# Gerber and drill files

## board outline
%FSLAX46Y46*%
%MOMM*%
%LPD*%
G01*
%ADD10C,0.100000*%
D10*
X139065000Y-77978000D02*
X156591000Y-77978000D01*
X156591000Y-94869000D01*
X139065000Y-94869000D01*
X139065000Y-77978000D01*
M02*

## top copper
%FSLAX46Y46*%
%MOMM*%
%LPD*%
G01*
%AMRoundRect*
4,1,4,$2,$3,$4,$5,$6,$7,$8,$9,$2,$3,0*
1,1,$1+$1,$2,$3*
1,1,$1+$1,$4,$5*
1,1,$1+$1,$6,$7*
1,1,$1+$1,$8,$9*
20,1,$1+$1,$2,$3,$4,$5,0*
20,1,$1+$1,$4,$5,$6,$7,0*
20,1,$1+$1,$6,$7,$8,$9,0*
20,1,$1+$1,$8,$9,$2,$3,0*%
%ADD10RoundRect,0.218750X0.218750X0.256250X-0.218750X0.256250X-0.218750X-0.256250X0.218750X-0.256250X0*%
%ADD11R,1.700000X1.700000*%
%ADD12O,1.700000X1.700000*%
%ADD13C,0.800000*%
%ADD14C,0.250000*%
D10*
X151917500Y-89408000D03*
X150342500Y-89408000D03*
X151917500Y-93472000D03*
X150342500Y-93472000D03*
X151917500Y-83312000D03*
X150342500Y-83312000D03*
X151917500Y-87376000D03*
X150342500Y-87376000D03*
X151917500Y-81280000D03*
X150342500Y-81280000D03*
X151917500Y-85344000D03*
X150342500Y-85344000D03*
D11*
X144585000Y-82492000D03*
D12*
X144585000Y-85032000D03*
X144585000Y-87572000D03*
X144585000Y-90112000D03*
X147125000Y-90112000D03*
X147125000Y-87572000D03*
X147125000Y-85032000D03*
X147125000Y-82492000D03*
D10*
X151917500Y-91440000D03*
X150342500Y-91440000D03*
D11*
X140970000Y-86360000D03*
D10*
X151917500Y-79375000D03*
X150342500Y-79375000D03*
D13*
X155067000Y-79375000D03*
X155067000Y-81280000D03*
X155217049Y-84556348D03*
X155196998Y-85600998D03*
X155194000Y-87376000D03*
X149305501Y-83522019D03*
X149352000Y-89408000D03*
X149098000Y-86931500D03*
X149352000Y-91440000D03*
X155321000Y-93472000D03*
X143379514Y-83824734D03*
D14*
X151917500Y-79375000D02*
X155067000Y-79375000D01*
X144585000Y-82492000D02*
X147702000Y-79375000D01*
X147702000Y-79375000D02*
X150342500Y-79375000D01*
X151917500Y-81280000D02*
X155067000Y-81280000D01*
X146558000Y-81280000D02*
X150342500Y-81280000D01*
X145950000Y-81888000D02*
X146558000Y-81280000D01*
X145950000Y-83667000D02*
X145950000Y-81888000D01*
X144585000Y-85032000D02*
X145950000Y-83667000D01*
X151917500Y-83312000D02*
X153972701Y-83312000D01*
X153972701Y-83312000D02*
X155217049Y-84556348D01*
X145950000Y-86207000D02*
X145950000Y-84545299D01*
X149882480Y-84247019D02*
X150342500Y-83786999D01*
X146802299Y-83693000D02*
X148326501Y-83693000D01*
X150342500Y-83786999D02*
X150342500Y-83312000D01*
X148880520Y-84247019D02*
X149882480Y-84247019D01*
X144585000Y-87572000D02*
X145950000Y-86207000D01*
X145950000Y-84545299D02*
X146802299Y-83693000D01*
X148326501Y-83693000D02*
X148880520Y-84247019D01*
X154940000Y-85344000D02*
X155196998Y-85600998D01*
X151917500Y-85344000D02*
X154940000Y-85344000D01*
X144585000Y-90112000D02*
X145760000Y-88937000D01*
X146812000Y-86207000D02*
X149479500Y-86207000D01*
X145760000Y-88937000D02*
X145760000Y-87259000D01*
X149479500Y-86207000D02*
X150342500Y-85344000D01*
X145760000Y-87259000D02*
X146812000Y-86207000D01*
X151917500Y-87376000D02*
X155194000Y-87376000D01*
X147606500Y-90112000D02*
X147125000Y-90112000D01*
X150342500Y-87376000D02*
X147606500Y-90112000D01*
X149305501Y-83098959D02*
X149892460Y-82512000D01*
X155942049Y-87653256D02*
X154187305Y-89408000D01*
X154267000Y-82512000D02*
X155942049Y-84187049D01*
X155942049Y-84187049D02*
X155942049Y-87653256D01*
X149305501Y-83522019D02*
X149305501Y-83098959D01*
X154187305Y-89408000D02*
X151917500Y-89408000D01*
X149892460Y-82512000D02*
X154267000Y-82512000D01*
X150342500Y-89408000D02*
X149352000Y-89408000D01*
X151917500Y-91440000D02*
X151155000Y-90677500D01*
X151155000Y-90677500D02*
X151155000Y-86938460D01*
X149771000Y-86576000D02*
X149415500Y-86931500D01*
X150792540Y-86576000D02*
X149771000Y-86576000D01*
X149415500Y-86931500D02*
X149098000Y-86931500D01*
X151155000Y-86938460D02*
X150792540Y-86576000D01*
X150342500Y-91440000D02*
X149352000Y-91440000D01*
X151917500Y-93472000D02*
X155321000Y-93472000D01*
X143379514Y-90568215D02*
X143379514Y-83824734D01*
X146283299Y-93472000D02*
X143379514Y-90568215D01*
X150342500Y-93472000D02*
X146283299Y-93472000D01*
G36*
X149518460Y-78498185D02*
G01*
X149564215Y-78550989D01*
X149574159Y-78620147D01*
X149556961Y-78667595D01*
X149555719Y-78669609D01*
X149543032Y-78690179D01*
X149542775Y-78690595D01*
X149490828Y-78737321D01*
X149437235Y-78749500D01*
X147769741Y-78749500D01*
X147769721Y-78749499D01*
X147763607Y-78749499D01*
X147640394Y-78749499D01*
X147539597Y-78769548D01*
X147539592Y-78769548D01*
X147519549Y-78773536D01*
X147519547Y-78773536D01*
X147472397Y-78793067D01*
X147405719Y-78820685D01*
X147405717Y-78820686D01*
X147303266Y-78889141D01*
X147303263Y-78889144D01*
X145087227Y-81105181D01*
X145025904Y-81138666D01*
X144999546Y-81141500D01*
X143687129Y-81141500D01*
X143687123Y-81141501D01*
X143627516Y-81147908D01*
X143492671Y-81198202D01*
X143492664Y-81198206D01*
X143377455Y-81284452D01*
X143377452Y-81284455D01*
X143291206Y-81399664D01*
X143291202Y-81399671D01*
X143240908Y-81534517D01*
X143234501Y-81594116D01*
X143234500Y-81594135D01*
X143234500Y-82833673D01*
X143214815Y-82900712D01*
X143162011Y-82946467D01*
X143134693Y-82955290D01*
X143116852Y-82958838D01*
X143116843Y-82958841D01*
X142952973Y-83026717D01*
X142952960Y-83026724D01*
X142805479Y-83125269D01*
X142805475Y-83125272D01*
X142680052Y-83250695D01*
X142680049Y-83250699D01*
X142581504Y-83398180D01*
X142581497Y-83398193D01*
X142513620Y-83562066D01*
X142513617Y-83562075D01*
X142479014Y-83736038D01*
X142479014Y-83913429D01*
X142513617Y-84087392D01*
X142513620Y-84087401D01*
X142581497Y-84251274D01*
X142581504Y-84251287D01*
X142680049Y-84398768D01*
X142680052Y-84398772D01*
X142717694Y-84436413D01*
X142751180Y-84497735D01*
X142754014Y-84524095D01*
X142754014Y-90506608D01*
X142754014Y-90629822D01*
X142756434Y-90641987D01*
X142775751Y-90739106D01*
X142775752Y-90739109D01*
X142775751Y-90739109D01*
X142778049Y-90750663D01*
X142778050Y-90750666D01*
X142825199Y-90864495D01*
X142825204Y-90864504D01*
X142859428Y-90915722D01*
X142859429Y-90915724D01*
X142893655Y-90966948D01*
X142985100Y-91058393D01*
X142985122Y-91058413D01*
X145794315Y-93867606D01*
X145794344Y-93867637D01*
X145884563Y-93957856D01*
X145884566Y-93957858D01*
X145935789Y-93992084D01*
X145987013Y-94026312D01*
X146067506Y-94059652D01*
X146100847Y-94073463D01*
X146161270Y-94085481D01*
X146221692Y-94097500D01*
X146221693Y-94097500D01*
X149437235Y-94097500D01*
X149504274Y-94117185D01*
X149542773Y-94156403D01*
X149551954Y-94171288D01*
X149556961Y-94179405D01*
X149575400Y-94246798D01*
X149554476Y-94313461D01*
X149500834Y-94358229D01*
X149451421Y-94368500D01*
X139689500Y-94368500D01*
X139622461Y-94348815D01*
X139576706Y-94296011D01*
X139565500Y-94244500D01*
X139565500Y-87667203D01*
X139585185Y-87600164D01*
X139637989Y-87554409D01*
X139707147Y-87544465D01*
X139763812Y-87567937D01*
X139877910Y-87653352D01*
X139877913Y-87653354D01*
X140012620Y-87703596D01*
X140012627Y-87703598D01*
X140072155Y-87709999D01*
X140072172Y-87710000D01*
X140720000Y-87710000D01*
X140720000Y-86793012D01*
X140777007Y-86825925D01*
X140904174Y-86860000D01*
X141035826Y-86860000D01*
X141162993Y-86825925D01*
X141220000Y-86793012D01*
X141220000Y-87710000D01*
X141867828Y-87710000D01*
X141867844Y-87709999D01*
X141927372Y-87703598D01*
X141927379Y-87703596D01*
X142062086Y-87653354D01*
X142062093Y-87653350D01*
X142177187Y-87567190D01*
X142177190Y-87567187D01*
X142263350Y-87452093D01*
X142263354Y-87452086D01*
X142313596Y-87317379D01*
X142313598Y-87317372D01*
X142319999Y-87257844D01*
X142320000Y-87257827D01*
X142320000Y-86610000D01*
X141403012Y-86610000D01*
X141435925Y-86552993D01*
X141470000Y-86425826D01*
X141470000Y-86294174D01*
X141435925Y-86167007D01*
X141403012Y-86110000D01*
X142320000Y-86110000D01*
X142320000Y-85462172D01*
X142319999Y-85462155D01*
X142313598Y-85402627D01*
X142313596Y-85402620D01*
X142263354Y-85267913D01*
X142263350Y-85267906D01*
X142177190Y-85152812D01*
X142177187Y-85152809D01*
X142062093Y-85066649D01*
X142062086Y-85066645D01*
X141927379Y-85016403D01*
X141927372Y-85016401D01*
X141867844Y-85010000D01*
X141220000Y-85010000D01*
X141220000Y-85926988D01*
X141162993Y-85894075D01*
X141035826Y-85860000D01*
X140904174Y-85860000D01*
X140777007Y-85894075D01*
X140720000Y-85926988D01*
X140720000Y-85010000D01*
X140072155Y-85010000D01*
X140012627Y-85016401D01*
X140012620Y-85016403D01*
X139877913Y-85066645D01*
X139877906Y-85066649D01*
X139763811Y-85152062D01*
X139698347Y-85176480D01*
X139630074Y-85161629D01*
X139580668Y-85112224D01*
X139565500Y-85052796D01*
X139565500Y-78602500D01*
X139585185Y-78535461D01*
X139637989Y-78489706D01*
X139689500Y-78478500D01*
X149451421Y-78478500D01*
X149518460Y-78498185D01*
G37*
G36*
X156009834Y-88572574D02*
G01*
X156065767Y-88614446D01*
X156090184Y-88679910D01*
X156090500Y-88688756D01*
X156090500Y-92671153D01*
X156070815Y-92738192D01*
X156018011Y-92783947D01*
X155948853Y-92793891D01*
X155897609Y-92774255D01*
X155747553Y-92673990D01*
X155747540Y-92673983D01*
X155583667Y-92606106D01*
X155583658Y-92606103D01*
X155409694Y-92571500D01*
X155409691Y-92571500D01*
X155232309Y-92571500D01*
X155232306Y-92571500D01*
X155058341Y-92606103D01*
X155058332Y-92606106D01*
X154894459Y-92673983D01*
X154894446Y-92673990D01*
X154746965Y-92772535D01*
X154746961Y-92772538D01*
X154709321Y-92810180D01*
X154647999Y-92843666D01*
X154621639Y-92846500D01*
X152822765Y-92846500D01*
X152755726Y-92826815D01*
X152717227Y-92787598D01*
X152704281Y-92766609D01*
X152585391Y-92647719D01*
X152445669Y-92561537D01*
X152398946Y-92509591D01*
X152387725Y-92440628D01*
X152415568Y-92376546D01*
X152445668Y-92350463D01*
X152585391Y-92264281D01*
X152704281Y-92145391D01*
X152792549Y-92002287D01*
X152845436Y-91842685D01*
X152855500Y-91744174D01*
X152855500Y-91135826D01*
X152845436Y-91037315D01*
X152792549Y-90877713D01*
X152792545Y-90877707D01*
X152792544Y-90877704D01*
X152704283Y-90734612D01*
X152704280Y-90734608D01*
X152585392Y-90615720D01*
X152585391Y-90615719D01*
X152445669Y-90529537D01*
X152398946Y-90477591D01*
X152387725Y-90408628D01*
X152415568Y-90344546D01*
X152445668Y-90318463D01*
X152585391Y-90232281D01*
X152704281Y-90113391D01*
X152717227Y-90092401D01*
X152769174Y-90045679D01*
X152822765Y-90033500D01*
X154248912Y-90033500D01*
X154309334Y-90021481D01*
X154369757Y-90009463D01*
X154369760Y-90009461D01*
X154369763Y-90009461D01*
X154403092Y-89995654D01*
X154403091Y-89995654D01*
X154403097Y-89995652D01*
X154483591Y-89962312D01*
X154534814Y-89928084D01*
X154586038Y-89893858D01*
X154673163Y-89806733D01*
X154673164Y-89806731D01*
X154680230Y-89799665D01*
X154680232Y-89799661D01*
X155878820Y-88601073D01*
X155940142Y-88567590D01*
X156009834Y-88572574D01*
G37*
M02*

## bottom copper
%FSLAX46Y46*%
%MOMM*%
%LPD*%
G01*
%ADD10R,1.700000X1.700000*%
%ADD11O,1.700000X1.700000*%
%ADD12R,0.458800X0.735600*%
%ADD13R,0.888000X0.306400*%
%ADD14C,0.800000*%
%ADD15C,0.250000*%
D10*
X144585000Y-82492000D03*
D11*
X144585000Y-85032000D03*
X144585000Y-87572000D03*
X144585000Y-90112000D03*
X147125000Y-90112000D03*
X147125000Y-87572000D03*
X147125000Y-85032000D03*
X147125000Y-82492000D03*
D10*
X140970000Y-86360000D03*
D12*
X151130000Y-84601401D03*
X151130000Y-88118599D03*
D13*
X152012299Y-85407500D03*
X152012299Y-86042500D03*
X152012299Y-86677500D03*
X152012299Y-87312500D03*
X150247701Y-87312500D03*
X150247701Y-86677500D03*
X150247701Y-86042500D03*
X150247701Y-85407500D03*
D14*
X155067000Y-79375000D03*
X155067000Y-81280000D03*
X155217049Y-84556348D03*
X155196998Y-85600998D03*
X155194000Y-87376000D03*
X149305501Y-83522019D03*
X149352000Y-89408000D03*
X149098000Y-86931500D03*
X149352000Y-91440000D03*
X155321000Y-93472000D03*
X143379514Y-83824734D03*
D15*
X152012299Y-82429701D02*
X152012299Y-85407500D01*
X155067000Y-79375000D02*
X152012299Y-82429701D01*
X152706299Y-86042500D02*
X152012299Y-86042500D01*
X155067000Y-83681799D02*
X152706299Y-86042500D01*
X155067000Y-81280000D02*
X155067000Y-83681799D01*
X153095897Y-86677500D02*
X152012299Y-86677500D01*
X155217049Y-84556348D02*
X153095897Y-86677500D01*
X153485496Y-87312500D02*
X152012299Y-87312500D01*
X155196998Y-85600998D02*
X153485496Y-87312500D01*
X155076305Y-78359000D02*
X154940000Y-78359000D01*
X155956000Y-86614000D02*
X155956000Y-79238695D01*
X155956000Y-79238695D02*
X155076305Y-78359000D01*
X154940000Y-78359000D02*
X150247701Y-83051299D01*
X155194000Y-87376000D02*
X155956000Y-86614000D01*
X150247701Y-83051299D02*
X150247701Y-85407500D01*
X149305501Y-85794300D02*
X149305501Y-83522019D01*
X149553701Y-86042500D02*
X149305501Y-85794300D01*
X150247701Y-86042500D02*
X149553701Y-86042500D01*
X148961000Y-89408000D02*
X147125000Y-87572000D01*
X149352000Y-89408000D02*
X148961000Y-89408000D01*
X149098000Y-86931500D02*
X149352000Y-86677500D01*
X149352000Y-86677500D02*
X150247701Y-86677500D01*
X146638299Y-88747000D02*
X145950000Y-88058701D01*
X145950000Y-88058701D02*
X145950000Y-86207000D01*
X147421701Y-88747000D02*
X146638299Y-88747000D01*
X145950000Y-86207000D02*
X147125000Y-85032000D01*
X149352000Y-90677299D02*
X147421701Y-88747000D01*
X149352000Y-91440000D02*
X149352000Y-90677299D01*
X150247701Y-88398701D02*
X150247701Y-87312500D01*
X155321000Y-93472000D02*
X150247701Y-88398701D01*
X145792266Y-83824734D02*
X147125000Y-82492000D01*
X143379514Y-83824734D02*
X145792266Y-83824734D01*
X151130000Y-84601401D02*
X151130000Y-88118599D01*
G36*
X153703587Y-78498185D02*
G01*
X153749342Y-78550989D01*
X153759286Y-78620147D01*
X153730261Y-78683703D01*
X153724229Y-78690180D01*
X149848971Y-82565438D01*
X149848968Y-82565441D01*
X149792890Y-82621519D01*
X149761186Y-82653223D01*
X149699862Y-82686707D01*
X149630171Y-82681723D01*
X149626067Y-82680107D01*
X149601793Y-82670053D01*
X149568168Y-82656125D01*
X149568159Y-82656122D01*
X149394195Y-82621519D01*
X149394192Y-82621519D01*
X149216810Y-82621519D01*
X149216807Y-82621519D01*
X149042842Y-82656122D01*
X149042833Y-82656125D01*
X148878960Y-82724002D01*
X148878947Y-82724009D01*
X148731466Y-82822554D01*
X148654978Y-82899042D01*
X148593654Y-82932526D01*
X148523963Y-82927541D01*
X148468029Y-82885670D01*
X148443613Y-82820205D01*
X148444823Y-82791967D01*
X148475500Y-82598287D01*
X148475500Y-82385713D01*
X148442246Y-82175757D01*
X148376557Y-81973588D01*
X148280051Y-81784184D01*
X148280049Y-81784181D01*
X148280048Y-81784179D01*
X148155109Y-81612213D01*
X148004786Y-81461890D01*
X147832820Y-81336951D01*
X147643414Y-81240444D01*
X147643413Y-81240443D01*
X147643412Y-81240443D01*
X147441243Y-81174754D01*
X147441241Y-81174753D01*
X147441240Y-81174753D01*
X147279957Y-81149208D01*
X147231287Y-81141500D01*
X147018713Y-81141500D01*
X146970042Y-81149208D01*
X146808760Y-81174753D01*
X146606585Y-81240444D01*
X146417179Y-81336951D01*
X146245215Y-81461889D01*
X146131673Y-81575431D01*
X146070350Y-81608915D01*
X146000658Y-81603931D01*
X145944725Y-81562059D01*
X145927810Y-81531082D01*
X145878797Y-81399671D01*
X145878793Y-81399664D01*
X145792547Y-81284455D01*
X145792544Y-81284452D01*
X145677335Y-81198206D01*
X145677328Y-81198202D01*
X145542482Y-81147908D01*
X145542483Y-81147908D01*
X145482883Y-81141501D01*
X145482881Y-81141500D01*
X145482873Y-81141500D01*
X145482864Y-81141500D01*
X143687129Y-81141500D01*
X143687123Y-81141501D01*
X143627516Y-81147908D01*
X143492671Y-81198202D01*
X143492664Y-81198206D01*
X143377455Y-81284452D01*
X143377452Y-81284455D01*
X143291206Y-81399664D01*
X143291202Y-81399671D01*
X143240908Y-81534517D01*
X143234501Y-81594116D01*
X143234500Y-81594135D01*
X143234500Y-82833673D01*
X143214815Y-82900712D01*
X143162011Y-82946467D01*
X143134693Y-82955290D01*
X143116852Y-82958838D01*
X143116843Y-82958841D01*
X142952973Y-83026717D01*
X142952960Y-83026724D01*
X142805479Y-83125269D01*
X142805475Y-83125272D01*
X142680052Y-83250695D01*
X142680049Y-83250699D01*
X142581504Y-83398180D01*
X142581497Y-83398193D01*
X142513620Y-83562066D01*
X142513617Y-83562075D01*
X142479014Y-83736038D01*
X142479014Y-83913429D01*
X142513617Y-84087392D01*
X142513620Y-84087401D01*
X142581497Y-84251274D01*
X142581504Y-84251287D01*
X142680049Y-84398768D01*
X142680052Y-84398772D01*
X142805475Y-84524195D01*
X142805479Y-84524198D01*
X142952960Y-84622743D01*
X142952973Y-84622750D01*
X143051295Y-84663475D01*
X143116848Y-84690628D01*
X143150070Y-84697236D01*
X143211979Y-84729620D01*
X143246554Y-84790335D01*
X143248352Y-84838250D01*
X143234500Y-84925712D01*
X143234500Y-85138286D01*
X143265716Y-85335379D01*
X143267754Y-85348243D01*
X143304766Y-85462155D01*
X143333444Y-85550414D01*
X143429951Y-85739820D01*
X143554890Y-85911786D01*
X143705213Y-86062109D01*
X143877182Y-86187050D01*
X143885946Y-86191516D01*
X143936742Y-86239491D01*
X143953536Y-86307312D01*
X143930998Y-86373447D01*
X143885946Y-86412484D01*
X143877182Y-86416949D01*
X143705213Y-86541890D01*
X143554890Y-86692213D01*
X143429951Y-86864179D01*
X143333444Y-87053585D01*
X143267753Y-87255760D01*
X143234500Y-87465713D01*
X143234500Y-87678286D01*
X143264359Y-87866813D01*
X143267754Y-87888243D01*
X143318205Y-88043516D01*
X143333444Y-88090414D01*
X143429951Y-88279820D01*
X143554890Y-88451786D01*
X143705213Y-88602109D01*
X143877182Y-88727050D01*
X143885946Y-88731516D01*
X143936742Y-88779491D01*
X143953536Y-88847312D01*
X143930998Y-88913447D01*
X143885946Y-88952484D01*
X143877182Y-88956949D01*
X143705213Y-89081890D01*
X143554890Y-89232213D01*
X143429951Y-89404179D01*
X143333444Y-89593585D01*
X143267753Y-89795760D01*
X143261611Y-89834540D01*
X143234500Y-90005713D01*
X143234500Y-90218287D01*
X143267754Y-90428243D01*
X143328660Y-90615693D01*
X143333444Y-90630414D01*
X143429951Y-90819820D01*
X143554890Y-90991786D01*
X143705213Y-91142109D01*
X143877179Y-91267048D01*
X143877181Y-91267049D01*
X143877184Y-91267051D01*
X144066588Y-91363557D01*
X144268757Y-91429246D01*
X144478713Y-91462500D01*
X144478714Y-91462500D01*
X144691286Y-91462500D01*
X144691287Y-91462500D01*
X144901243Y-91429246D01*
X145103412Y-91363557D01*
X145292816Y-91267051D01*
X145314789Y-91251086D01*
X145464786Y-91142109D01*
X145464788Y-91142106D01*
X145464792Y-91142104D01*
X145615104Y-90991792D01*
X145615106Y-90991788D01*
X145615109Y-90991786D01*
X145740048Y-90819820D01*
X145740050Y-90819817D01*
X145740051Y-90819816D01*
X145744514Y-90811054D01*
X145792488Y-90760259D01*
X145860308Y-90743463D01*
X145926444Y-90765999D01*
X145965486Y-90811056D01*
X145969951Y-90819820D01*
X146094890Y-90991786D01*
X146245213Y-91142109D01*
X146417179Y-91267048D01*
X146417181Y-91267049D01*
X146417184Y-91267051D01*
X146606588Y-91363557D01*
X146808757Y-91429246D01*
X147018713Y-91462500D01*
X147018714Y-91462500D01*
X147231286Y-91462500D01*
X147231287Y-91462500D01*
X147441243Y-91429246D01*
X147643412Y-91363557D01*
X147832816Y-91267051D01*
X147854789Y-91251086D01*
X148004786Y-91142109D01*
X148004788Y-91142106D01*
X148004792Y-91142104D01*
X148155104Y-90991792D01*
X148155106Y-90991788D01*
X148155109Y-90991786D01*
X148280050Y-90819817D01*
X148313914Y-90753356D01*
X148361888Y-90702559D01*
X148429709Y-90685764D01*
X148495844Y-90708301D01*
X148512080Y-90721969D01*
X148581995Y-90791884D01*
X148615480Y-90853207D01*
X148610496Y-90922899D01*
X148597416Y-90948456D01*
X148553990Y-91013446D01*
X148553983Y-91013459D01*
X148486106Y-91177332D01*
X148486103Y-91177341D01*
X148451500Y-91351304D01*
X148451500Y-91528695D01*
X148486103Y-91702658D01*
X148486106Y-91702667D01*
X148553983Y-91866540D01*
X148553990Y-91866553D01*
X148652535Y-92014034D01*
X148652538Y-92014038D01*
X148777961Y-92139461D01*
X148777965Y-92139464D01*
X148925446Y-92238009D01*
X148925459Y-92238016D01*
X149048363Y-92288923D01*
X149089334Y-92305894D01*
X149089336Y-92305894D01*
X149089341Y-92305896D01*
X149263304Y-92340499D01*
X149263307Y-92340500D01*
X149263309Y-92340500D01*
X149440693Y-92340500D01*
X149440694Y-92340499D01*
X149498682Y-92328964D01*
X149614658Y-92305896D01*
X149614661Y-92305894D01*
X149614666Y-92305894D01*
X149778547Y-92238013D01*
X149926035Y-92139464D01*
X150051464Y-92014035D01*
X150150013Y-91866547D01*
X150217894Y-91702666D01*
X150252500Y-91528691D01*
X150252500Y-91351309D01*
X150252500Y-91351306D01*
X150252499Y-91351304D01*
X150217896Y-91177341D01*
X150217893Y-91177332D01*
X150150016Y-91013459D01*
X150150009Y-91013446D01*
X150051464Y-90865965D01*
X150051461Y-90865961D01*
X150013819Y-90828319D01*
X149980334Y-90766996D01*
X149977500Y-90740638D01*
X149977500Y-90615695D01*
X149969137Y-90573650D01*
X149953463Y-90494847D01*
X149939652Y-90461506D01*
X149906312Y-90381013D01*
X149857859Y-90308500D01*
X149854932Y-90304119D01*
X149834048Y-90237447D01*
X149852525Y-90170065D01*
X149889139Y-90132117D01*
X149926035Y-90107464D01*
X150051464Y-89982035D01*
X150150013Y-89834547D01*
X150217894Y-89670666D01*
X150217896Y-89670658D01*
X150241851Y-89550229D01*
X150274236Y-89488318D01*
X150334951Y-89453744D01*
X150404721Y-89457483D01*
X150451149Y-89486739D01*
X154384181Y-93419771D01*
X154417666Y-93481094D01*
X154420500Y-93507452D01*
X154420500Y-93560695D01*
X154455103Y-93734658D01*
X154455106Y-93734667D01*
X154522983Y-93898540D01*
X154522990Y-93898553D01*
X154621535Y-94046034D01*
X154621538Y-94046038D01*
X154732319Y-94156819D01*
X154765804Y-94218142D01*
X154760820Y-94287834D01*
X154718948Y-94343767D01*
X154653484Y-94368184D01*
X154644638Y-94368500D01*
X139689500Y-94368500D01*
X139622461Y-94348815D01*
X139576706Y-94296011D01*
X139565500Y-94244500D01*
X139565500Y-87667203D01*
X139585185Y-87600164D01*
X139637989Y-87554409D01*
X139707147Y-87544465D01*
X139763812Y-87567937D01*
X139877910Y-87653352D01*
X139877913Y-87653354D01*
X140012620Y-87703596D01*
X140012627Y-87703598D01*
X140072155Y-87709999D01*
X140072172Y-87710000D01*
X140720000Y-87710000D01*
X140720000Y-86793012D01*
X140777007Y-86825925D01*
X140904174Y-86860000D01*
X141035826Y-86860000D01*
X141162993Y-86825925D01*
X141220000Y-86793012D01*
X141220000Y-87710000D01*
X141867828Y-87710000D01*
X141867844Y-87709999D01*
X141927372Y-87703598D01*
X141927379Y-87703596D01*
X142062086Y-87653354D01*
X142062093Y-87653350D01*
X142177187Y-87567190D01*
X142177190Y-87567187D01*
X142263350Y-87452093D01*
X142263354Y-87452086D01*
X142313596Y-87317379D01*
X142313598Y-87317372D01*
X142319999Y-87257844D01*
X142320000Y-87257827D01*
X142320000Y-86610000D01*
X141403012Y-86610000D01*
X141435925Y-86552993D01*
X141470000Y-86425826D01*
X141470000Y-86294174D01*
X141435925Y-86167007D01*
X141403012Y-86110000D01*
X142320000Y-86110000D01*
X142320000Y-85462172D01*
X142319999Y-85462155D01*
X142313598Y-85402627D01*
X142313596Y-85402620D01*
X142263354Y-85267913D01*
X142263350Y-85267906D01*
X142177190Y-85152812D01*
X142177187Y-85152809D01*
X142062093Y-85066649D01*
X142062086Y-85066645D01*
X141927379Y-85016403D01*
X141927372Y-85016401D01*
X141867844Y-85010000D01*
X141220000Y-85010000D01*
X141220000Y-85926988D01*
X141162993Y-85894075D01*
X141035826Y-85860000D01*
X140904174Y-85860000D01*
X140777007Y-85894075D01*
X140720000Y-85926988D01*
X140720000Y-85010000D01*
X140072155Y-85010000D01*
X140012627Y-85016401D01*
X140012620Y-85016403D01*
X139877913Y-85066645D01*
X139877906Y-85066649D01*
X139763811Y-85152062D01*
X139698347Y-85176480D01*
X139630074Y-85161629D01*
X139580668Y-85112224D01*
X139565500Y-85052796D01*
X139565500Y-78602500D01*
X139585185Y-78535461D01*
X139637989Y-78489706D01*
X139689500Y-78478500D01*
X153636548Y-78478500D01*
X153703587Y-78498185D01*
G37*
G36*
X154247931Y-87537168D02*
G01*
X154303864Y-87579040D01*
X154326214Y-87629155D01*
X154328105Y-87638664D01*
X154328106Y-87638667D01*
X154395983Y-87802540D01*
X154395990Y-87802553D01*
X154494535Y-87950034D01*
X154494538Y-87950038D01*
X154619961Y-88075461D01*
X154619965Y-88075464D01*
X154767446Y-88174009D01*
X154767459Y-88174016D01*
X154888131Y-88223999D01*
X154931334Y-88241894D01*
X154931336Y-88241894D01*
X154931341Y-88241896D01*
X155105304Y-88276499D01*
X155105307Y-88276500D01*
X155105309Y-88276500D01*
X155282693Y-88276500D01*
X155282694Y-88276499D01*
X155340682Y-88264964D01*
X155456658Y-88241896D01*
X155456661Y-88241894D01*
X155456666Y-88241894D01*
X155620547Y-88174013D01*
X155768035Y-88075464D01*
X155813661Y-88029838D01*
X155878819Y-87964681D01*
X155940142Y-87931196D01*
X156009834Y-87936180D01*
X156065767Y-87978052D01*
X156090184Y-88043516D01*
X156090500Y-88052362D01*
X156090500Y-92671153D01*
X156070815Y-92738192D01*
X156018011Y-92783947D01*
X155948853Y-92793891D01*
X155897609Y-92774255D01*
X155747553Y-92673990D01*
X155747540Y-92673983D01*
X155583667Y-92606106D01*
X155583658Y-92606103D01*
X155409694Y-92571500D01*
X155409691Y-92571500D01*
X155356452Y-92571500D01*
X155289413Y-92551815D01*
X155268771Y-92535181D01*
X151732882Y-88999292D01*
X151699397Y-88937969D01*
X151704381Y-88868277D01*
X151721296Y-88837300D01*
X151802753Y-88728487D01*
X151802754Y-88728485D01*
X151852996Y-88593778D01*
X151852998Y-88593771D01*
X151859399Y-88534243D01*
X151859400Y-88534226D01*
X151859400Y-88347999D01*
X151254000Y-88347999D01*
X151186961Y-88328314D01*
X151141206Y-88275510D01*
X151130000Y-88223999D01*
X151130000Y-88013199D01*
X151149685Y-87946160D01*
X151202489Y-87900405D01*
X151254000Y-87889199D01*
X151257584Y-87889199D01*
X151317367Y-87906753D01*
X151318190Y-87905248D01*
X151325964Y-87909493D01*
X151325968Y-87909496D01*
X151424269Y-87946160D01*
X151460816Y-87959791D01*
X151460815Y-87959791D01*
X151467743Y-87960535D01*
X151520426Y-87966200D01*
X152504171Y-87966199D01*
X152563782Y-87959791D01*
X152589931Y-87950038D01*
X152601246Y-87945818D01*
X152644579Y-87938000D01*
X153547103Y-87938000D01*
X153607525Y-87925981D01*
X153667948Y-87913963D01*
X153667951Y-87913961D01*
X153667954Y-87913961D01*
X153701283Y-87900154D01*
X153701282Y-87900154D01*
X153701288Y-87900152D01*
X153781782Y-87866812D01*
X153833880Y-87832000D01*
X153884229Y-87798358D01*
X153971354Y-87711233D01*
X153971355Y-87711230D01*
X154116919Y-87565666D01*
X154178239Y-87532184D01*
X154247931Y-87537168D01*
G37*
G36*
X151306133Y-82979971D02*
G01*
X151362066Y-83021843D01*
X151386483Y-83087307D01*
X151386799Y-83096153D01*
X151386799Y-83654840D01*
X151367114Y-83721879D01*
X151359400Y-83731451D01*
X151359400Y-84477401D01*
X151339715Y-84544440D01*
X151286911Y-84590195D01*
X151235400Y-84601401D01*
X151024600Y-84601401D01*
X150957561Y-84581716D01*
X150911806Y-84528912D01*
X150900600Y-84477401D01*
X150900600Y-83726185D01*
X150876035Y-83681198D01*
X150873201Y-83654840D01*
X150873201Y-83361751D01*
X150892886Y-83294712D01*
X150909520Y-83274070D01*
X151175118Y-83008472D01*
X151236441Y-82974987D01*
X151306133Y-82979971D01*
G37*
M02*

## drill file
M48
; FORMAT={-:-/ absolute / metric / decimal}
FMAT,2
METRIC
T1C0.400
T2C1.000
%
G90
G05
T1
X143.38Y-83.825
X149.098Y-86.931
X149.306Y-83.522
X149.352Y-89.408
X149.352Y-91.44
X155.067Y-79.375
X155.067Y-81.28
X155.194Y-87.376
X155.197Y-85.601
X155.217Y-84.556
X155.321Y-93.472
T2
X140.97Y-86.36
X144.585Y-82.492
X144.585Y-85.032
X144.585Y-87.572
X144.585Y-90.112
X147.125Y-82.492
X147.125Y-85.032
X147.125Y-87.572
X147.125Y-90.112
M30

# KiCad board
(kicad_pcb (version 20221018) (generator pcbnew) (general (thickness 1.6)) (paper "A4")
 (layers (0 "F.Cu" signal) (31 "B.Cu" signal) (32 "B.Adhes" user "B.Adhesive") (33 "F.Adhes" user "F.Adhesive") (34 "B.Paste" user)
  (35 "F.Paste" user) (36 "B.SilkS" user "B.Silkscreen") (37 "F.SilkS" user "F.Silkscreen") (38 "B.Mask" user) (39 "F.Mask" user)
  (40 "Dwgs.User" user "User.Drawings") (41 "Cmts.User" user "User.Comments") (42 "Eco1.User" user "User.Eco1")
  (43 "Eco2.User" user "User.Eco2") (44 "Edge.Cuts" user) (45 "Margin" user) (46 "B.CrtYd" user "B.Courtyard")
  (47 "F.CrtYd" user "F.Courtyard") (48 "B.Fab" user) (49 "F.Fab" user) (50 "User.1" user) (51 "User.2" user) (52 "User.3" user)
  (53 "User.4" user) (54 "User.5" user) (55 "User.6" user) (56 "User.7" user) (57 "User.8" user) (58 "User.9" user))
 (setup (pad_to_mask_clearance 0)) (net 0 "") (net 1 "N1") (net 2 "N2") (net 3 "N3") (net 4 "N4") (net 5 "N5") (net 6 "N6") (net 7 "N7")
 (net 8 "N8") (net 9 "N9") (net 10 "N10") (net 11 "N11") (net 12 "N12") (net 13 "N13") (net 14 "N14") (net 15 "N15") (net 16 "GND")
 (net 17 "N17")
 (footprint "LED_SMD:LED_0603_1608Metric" (layer "F.Cu") (at 151.13 89.408 180)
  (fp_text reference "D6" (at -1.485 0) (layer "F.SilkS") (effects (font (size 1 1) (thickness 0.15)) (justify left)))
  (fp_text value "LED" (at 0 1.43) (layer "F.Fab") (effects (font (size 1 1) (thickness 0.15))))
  (pad "1" smd roundrect (at -0.7875 0 180) (size 0.875 0.95) (layers "F.Cu" "F.Paste" "F.Mask") (roundrect_rratio 0.25) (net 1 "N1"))
  (pad "2" smd roundrect (at 0.7875 0 180) (size 0.875 0.95) (layers "F.Cu" "F.Paste" "F.Mask") (roundrect_rratio 0.25) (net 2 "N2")))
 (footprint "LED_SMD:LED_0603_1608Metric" (layer "F.Cu") (at 151.13 93.472 180)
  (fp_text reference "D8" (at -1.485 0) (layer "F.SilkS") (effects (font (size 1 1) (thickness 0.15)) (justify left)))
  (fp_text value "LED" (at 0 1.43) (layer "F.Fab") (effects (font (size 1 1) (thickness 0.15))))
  (pad "1" smd roundrect (at -0.7875 0 180) (size 0.875 0.95) (layers "F.Cu" "F.Paste" "F.Mask") (roundrect_rratio 0.25) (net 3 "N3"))
  (pad "2" smd roundrect (at 0.7875 0 180) (size 0.875 0.95) (layers "F.Cu" "F.Paste" "F.Mask") (roundrect_rratio 0.25) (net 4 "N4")))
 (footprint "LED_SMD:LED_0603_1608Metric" (layer "F.Cu") (at 151.13 83.312 180)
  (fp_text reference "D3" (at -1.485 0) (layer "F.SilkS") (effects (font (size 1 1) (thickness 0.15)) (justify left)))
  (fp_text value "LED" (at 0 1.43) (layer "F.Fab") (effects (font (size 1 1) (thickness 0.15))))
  (pad "1" smd roundrect (at -0.7875 0 180) (size 0.875 0.95) (layers "F.Cu" "F.Paste" "F.Mask") (roundrect_rratio 0.25) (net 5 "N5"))
  (pad "2" smd roundrect (at 0.7875 0 180) (size 0.875 0.95) (layers "F.Cu" "F.Paste" "F.Mask") (roundrect_rratio 0.25) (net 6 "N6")))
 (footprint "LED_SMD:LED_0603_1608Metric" (layer "F.Cu") (at 151.13 87.376 180)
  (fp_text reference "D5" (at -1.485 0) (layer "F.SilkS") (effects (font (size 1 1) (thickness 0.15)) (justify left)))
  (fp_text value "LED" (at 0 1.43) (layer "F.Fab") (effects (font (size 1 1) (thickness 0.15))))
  (pad "1" smd roundrect (at -0.7875 0 180) (size 0.875 0.95) (layers "F.Cu" "F.Paste" "F.Mask") (roundrect_rratio 0.25) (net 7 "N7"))
  (pad "2" smd roundrect (at 0.7875 0 180) (size 0.875 0.95) (layers "F.Cu" "F.Paste" "F.Mask") (roundrect_rratio 0.25) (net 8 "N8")))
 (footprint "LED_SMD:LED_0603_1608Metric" (layer "F.Cu") (at 151.13 81.28 180)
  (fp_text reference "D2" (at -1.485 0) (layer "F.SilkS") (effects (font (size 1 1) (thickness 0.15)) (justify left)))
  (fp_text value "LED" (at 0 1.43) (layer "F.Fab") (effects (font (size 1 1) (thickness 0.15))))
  (pad "1" smd roundrect (at -0.7875 0 180) (size 0.875 0.95) (layers "F.Cu" "F.Paste" "F.Mask") (roundrect_rratio 0.25) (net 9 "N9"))
  (pad "2" smd roundrect (at 0.7875 0 180) (size 0.875 0.95) (layers "F.Cu" "F.Paste" "F.Mask") (roundrect_rratio 0.25) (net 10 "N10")))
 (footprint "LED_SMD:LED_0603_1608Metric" (layer "F.Cu") (at 151.13 85.344 180)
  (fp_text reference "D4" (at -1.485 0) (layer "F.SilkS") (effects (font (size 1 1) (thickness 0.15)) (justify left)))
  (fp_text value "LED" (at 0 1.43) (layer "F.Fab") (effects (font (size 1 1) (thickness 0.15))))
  (pad "1" smd roundrect (at -0.7875 0 180) (size 0.875 0.95) (layers "F.Cu" "F.Paste" "F.Mask") (roundrect_rratio 0.25) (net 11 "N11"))
  (pad "2" smd roundrect (at 0.7875 0 180) (size 0.875 0.95) (layers "F.Cu" "F.Paste" "F.Mask") (roundrect_rratio 0.25) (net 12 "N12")))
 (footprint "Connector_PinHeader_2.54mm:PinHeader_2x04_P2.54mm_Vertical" (layer "F.Cu") (at 144.585 82.492)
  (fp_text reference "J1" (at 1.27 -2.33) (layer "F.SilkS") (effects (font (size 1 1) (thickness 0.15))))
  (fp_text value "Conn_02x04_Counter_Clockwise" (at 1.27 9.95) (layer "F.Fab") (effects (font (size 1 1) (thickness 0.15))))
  (pad "1" thru_hole rect (at 0 0) (size 1.7 1.7) (drill 1) (layers "*.Cu" "*.Mask") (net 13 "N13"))
  (pad "2" thru_hole oval (at 0 2.54) (size 1.7 1.7) (drill 1) (layers "*.Cu" "*.Mask") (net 10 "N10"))
  (pad "3" thru_hole oval (at 0 5.08) (size 1.7 1.7) (drill 1) (layers "*.Cu" "*.Mask") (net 6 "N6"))
  (pad "4" thru_hole oval (at 0 7.62) (size 1.7 1.7) (drill 1) (layers "*.Cu" "*.Mask") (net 12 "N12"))
  (pad "5" thru_hole oval (at 2.54 7.62) (size 1.7 1.7) (drill 1) (layers "*.Cu" "*.Mask") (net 8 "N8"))
  (pad "6" thru_hole oval (at 2.54 5.08) (size 1.7 1.7) (drill 1) (layers "*.Cu" "*.Mask") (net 2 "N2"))
  (pad "7" thru_hole oval (at 2.54 2.54) (size 1.7 1.7) (drill 1) (layers "*.Cu" "*.Mask") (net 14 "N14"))
  (pad "8" thru_hole oval (at 2.54 0) (size 1.7 1.7) (drill 1) (layers "*.Cu" "*.Mask") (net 4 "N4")))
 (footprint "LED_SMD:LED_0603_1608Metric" (layer "F.Cu") (at 151.13 91.44 180)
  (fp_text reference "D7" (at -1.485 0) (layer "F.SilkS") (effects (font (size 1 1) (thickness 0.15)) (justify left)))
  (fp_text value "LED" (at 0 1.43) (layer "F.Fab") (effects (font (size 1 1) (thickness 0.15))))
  (pad "1" smd roundrect (at -0.7875 0 180) (size 0.875 0.95) (layers "F.Cu" "F.Paste" "F.Mask") (roundrect_rratio 0.25) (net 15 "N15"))
  (pad "2" smd roundrect (at 0.7875 0 180) (size 0.875 0.95) (layers "F.Cu" "F.Paste" "F.Mask") (roundrect_rratio 0.25) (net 14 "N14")))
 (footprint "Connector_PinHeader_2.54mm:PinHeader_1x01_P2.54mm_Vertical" (layer "F.Cu") (at 140.97 86.36)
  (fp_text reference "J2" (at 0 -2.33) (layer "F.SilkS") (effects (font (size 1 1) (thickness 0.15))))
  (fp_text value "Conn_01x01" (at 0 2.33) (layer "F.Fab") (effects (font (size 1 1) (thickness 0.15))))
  (pad "1" thru_hole rect (at 0 0) (size 1.7 1.7) (drill 1) (layers "*.Cu" "*.Mask") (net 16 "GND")))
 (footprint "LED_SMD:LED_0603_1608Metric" (layer "F.Cu") (at 151.13 79.375 180)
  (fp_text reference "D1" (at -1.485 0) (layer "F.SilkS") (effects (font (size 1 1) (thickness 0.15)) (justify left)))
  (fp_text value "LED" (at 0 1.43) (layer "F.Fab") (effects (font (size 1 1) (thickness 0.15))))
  (pad "1" smd roundrect (at -0.7875 0 180) (size 0.875 0.95) (layers "F.Cu" "F.Paste" "F.Mask") (roundrect_rratio 0.25) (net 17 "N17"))
  (pad "2" smd roundrect (at 0.7875 0 180) (size 0.875 0.95) (layers "F.Cu" "F.Paste" "F.Mask") (roundrect_rratio 0.25) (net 13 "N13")))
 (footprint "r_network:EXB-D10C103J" (layer "B.Cu") (at 151.13 86.36 -90)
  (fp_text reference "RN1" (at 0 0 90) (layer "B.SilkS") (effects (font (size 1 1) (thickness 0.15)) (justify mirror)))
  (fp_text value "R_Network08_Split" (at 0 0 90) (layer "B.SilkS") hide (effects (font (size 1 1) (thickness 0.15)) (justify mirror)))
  (pad "1" smd rect (at -1.758599 0 270) (size 0.7356 0.4588) (layers "B.Cu" "B.Paste" "B.Mask") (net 16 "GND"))
  (pad "1" smd rect (at 1.758599 0 270) (size 0.7356 0.4588) (layers "B.Cu" "B.Paste" "B.Mask") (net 16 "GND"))
  (pad "2" smd rect (at -0.9525 -0.882299 180) (size 0.888 0.3064) (layers "B.Cu" "B.Paste" "B.Mask") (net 17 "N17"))
  (pad "3" smd rect (at -0.3175 -0.882299 180) (size 0.888 0.3064) (layers "B.Cu" "B.Paste" "B.Mask") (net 9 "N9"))
  (pad "4" smd rect (at 0.3175 -0.882299 180) (size 0.888 0.3064) (layers "B.Cu" "B.Paste" "B.Mask") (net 5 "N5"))
  (pad "5" smd rect (at 0.9525 -0.882299 180) (size 0.888 0.3064) (layers "B.Cu" "B.Paste" "B.Mask") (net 11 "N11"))
  (pad "6" smd rect (at 0.9525 0.882299 180) (size 0.888 0.3064) (layers "B.Cu" "B.Paste" "B.Mask") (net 3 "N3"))
  (pad "7" smd rect (at 0.3175 0.882299 180) (size 0.888 0.3064) (layers "B.Cu" "B.Paste" "B.Mask") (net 15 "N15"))
  (pad "8" smd rect (at -0.3175 0.882299 180) (size 0.888 0.3064) (layers "B.Cu" "B.Paste" "B.Mask") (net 1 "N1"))
  (pad "9" smd rect (at -0.9525 0.882299 180) (size 0.888 0.3064) (layers "B.Cu" "B.Paste" "B.Mask") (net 7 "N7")))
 (gr_rect (start 139.065 77.978) (end 156.591 94.869) (stroke (width 0.1) (type default)) (fill none) (layer "Edge.Cuts"))
 (segment (start 151.9175 79.375) (end 155.067 79.375) (width 0.25) (layer "F.Cu") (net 17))
 (via (at 155.067 79.375) (size 0.8) (drill 0.4) (layers "F.Cu" "B.Cu") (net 17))
 (segment (start 152.012299 82.429701) (end 152.012299 85.4075) (width 0.25) (layer "B.Cu") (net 17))
 (segment (start 155.067 79.375) (end 152.012299 82.429701) (width 0.25) (layer "B.Cu") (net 17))
 (segment (start 144.585 82.492) (end 147.702 79.375) (width 0.25) (layer "F.Cu") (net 13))
 (segment (start 147.702 79.375) (end 150.3425 79.375) (width 0.25) (layer "F.Cu") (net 13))
 (segment (start 151.9175 81.28) (end 155.067 81.28) (width 0.25) (layer "F.Cu") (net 9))
 (via (at 155.067 81.28) (size 0.8) (drill 0.4) (layers "F.Cu" "B.Cu") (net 9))
 (segment (start 152.706299 86.0425) (end 152.012299 86.0425) (width 0.25) (layer "B.Cu") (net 9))
 (segment (start 155.067 83.681799) (end 152.706299 86.0425) (width 0.25) (layer "B.Cu") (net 9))
 (segment (start 155.067 81.28) (end 155.067 83.681799) (width 0.25) (layer "B.Cu") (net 9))
 (segment (start 146.558 81.28) (end 150.3425 81.28) (width 0.25) (layer "F.Cu") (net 10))
 (segment (start 145.95 81.888) (end 146.558 81.28) (width 0.25) (layer "F.Cu") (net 10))
 (segment (start 145.95 83.667) (end 145.95 81.888) (width 0.25) (layer "F.Cu") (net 10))
 (segment (start 144.585 85.032) (end 145.95 83.667) (width 0.25) (layer "F.Cu") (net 10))
 (segment (start 151.9175 83.312) (end 153.972701 83.312) (width 0.25) (layer "F.Cu") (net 5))
 (segment (start 153.972701 83.312) (end 155.217049 84.556348) (width 0.25) (layer "F.Cu") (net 5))
 (via (at 155.217049 84.556348) (size 0.8) (drill 0.4) (layers "F.Cu" "B.Cu") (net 5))
 (segment (start 153.095897 86.6775) (end 152.012299 86.6775) (width 0.25) (layer "B.Cu") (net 5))
 (segment (start 155.217049 84.556348) (end 153.095897 86.6775) (width 0.25) (layer "B.Cu") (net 5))
 (segment (start 145.95 86.207) (end 145.95 84.545299) (width 0.25) (layer "F.Cu") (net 6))
 (segment (start 149.88248 84.247019) (end 150.3425 83.786999) (width 0.25) (layer "F.Cu") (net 6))
 (segment (start 146.802299 83.693) (end 148.326501 83.693) (width 0.25) (layer "F.Cu") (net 6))
 (segment (start 150.3425 83.786999) (end 150.3425 83.312) (width 0.25) (layer "F.Cu") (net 6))
 (segment (start 148.88052 84.247019) (end 149.88248 84.247019) (width 0.25) (layer "F.Cu") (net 6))
 (segment (start 144.585 87.572) (end 145.95 86.207) (width 0.25) (layer "F.Cu") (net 6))
 (segment (start 145.95 84.545299) (end 146.802299 83.693) (width 0.25) (layer "F.Cu") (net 6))
 (segment (start 148.326501 83.693) (end 148.88052 84.247019) (width 0.25) (layer "F.Cu") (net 6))
 (segment (start 154.94 85.344) (end 155.196998 85.600998) (width 0.25) (layer "F.Cu") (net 11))
 (segment (start 151.9175 85.344) (end 154.94 85.344) (width 0.25) (layer "F.Cu") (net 11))
 (via (at 155.196998 85.600998) (size 0.8) (drill 0.4) (layers "F.Cu" "B.Cu") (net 11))
 (segment (start 153.485496 87.3125) (end 152.012299 87.3125) (width 0.25) (layer "B.Cu") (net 11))
 (segment (start 155.196998 85.600998) (end 153.485496 87.3125) (width 0.25) (layer "B.Cu") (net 11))
 (segment (start 144.585 90.112) (end 145.76 88.937) (width 0.25) (layer "F.Cu") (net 12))
 (segment (start 146.812 86.207) (end 149.4795 86.207) (width 0.25) (layer "F.Cu") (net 12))
 (segment (start 145.76 88.937) (end 145.76 87.259) (width 0.25) (layer "F.Cu") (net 12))
 (segment (start 149.4795 86.207) (end 150.3425 85.344) (width 0.25) (layer "F.Cu") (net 12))
 (segment (start 145.76 87.259) (end 146.812 86.207) (width 0.25) (layer "F.Cu") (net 12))
 (segment (start 151.9175 87.376) (end 155.194 87.376) (width 0.25) (layer "F.Cu") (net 7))
 (via (at 155.194 87.376) (size 0.8) (drill 0.4) (layers "F.Cu" "B.Cu") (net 7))
 (segment (start 155.076305 78.359) (end 154.94 78.359) (width 0.25) (layer "B.Cu") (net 7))
 (segment (start 155.956 86.614) (end 155.956 79.238695) (width 0.25) (layer "B.Cu") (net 7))
 (segment (start 155.956 79.238695) (end 155.076305 78.359) (width 0.25) (layer "B.Cu") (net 7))
 (segment (start 154.94 78.359) (end 150.247701 83.051299) (width 0.25) (layer "B.Cu") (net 7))
 (segment (start 155.194 87.376) (end 155.956 86.614) (width 0.25) (layer "B.Cu") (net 7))
 (segment (start 150.247701 83.051299) (end 150.247701 85.4075) (width 0.25) (layer "B.Cu") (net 7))
 (segment (start 147.6065 90.112) (end 147.125 90.112) (width 0.25) (layer "F.Cu") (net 8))
 (segment (start 150.3425 87.376) (end 147.6065 90.112) (width 0.25) (layer "F.Cu") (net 8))
 (segment (start 149.305501 83.098959) (end 149.89246 82.512) (width 0.25) (layer "F.Cu") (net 1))
 (segment (start 155.942049 87.653256) (end 154.187305 89.408) (width 0.25) (layer "F.Cu") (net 1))
 (segment (start 154.267 82.512) (end 155.942049 84.187049) (width 0.25) (layer "F.Cu") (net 1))
 (segment (start 155.942049 84.187049) (end 155.942049 87.653256) (width 0.25) (layer "F.Cu") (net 1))
 (segment (start 149.305501 83.522019) (end 149.305501 83.098959) (width 0.25) (layer "F.Cu") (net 1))
 (segment (start 154.187305 89.408) (end 151.9175 89.408) (width 0.25) (layer "F.Cu") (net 1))
 (segment (start 149.89246 82.512) (end 154.267 82.512) (width 0.25) (layer "F.Cu") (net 1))
 (via (at 149.305501 83.522019) (size 0.8) (drill 0.4) (layers "F.Cu" "B.Cu") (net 1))
 (segment (start 149.305501 85.7943) (end 149.305501 83.522019) (width 0.25) (layer "B.Cu") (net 1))
 (segment (start 149.553701 86.0425) (end 149.305501 85.7943) (width 0.25) (layer "B.Cu") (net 1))
 (segment (start 150.247701 86.0425) (end 149.553701 86.0425) (width 0.25) (layer "B.Cu") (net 1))
 (segment (start 150.3425 89.408) (end 149.352 89.408) (width 0.25) (layer "F.Cu") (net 2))
 (via (at 149.352 89.408) (size 0.8) (drill 0.4) (layers "F.Cu" "B.Cu") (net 2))
 (segment (start 148.961 89.408) (end 147.125 87.572) (width 0.25) (layer "B.Cu") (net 2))
 (segment (start 149.352 89.408) (end 148.961 89.408) (width 0.25) (layer "B.Cu") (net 2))
 (segment (start 151.9175 91.44) (end 151.155 90.6775) (width 0.25) (layer "F.Cu") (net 15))
 (segment (start 151.155 90.6775) (end 151.155 86.93846) (width 0.25) (layer "F.Cu") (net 15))
 (segment (start 149.771 86.576) (end 149.4155 86.9315) (width 0.25) (layer "F.Cu") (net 15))
 (segment (start 150.79254 86.576) (end 149.771 86.576) (width 0.25) (layer "F.Cu") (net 15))
 (segment (start 149.4155 86.9315) (end 149.098 86.9315) (width 0.25) (layer "F.Cu") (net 15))
 (segment (start 151.155 86.93846) (end 150.79254 86.576) (width 0.25) (layer "F.Cu") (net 15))
 (via (at 149.098 86.9315) (size 0.8) (drill 0.4) (layers "F.Cu" "B.Cu") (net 15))
 (segment (start 149.098 86.9315) (end 149.352 86.6775) (width 0.25) (layer "B.Cu") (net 15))
 (segment (start 149.352 86.6775) (end 150.247701 86.6775) (width 0.25) (layer "B.Cu") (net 15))
 (segment (start 150.3425 91.44) (end 149.352 91.44) (width 0.25) (layer "F.Cu") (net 14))
 (via (at 149.352 91.44) (size 0.8) (drill 0.4) (layers "F.Cu" "B.Cu") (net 14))
 (segment (start 146.638299 88.747) (end 145.95 88.058701) (width 0.25) (layer "B.Cu") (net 14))
 (segment (start 145.95 88.058701) (end 145.95 86.207) (width 0.25) (layer "B.Cu") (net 14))
 (segment (start 147.421701 88.747) (end 146.638299 88.747) (width 0.25) (layer "B.Cu") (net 14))
 (segment (start 145.95 86.207) (end 147.125 85.032) (width 0.25) (layer "B.Cu") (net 14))
 (segment (start 149.352 90.677299) (end 147.421701 88.747) (width 0.25) (layer "B.Cu") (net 14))
 (segment (start 149.352 91.44) (end 149.352 90.677299) (width 0.25) (layer "B.Cu") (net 14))
 (segment (start 151.9175 93.472) (end 155.321 93.472) (width 0.25) (layer "F.Cu") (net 3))
 (via (at 155.321 93.472) (size 0.8) (drill 0.4) (layers "F.Cu" "B.Cu") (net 3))
 (segment (start 150.247701 88.398701) (end 150.247701 87.3125) (width 0.25) (layer "B.Cu") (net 3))
 (segment (start 155.321 93.472) (end 150.247701 88.398701) (width 0.25) (layer "B.Cu") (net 3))
 (segment (start 143.379514 90.568215) (end 143.379514 83.824734) (width 0.25) (layer "F.Cu") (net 4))
 (segment (start 146.283299 93.472) (end 143.379514 90.568215) (width 0.25) (layer "F.Cu") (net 4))
 (segment (start 150.3425 93.472) (end 146.283299 93.472) (width 0.25) (layer "F.Cu") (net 4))
 (via (at 143.379514 83.824734) (size 0.8) (drill 0.4) (layers "F.Cu" "B.Cu") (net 4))
 (segment (start 145.792266 83.824734) (end 147.125 82.492) (width 0.25) (layer "B.Cu") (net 4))
 (segment (start 143.379514 83.824734) (end 145.792266 83.824734) (width 0.25) (layer "B.Cu") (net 4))
 (segment (start 151.13 84.601401) (end 151.13 88.118599) (width 0.25) (layer "B.Cu") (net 16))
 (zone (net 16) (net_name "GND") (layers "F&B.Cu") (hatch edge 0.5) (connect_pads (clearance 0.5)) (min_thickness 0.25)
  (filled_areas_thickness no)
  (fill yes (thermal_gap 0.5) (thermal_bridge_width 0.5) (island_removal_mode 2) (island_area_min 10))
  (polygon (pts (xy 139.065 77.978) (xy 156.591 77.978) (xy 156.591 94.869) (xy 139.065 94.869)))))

